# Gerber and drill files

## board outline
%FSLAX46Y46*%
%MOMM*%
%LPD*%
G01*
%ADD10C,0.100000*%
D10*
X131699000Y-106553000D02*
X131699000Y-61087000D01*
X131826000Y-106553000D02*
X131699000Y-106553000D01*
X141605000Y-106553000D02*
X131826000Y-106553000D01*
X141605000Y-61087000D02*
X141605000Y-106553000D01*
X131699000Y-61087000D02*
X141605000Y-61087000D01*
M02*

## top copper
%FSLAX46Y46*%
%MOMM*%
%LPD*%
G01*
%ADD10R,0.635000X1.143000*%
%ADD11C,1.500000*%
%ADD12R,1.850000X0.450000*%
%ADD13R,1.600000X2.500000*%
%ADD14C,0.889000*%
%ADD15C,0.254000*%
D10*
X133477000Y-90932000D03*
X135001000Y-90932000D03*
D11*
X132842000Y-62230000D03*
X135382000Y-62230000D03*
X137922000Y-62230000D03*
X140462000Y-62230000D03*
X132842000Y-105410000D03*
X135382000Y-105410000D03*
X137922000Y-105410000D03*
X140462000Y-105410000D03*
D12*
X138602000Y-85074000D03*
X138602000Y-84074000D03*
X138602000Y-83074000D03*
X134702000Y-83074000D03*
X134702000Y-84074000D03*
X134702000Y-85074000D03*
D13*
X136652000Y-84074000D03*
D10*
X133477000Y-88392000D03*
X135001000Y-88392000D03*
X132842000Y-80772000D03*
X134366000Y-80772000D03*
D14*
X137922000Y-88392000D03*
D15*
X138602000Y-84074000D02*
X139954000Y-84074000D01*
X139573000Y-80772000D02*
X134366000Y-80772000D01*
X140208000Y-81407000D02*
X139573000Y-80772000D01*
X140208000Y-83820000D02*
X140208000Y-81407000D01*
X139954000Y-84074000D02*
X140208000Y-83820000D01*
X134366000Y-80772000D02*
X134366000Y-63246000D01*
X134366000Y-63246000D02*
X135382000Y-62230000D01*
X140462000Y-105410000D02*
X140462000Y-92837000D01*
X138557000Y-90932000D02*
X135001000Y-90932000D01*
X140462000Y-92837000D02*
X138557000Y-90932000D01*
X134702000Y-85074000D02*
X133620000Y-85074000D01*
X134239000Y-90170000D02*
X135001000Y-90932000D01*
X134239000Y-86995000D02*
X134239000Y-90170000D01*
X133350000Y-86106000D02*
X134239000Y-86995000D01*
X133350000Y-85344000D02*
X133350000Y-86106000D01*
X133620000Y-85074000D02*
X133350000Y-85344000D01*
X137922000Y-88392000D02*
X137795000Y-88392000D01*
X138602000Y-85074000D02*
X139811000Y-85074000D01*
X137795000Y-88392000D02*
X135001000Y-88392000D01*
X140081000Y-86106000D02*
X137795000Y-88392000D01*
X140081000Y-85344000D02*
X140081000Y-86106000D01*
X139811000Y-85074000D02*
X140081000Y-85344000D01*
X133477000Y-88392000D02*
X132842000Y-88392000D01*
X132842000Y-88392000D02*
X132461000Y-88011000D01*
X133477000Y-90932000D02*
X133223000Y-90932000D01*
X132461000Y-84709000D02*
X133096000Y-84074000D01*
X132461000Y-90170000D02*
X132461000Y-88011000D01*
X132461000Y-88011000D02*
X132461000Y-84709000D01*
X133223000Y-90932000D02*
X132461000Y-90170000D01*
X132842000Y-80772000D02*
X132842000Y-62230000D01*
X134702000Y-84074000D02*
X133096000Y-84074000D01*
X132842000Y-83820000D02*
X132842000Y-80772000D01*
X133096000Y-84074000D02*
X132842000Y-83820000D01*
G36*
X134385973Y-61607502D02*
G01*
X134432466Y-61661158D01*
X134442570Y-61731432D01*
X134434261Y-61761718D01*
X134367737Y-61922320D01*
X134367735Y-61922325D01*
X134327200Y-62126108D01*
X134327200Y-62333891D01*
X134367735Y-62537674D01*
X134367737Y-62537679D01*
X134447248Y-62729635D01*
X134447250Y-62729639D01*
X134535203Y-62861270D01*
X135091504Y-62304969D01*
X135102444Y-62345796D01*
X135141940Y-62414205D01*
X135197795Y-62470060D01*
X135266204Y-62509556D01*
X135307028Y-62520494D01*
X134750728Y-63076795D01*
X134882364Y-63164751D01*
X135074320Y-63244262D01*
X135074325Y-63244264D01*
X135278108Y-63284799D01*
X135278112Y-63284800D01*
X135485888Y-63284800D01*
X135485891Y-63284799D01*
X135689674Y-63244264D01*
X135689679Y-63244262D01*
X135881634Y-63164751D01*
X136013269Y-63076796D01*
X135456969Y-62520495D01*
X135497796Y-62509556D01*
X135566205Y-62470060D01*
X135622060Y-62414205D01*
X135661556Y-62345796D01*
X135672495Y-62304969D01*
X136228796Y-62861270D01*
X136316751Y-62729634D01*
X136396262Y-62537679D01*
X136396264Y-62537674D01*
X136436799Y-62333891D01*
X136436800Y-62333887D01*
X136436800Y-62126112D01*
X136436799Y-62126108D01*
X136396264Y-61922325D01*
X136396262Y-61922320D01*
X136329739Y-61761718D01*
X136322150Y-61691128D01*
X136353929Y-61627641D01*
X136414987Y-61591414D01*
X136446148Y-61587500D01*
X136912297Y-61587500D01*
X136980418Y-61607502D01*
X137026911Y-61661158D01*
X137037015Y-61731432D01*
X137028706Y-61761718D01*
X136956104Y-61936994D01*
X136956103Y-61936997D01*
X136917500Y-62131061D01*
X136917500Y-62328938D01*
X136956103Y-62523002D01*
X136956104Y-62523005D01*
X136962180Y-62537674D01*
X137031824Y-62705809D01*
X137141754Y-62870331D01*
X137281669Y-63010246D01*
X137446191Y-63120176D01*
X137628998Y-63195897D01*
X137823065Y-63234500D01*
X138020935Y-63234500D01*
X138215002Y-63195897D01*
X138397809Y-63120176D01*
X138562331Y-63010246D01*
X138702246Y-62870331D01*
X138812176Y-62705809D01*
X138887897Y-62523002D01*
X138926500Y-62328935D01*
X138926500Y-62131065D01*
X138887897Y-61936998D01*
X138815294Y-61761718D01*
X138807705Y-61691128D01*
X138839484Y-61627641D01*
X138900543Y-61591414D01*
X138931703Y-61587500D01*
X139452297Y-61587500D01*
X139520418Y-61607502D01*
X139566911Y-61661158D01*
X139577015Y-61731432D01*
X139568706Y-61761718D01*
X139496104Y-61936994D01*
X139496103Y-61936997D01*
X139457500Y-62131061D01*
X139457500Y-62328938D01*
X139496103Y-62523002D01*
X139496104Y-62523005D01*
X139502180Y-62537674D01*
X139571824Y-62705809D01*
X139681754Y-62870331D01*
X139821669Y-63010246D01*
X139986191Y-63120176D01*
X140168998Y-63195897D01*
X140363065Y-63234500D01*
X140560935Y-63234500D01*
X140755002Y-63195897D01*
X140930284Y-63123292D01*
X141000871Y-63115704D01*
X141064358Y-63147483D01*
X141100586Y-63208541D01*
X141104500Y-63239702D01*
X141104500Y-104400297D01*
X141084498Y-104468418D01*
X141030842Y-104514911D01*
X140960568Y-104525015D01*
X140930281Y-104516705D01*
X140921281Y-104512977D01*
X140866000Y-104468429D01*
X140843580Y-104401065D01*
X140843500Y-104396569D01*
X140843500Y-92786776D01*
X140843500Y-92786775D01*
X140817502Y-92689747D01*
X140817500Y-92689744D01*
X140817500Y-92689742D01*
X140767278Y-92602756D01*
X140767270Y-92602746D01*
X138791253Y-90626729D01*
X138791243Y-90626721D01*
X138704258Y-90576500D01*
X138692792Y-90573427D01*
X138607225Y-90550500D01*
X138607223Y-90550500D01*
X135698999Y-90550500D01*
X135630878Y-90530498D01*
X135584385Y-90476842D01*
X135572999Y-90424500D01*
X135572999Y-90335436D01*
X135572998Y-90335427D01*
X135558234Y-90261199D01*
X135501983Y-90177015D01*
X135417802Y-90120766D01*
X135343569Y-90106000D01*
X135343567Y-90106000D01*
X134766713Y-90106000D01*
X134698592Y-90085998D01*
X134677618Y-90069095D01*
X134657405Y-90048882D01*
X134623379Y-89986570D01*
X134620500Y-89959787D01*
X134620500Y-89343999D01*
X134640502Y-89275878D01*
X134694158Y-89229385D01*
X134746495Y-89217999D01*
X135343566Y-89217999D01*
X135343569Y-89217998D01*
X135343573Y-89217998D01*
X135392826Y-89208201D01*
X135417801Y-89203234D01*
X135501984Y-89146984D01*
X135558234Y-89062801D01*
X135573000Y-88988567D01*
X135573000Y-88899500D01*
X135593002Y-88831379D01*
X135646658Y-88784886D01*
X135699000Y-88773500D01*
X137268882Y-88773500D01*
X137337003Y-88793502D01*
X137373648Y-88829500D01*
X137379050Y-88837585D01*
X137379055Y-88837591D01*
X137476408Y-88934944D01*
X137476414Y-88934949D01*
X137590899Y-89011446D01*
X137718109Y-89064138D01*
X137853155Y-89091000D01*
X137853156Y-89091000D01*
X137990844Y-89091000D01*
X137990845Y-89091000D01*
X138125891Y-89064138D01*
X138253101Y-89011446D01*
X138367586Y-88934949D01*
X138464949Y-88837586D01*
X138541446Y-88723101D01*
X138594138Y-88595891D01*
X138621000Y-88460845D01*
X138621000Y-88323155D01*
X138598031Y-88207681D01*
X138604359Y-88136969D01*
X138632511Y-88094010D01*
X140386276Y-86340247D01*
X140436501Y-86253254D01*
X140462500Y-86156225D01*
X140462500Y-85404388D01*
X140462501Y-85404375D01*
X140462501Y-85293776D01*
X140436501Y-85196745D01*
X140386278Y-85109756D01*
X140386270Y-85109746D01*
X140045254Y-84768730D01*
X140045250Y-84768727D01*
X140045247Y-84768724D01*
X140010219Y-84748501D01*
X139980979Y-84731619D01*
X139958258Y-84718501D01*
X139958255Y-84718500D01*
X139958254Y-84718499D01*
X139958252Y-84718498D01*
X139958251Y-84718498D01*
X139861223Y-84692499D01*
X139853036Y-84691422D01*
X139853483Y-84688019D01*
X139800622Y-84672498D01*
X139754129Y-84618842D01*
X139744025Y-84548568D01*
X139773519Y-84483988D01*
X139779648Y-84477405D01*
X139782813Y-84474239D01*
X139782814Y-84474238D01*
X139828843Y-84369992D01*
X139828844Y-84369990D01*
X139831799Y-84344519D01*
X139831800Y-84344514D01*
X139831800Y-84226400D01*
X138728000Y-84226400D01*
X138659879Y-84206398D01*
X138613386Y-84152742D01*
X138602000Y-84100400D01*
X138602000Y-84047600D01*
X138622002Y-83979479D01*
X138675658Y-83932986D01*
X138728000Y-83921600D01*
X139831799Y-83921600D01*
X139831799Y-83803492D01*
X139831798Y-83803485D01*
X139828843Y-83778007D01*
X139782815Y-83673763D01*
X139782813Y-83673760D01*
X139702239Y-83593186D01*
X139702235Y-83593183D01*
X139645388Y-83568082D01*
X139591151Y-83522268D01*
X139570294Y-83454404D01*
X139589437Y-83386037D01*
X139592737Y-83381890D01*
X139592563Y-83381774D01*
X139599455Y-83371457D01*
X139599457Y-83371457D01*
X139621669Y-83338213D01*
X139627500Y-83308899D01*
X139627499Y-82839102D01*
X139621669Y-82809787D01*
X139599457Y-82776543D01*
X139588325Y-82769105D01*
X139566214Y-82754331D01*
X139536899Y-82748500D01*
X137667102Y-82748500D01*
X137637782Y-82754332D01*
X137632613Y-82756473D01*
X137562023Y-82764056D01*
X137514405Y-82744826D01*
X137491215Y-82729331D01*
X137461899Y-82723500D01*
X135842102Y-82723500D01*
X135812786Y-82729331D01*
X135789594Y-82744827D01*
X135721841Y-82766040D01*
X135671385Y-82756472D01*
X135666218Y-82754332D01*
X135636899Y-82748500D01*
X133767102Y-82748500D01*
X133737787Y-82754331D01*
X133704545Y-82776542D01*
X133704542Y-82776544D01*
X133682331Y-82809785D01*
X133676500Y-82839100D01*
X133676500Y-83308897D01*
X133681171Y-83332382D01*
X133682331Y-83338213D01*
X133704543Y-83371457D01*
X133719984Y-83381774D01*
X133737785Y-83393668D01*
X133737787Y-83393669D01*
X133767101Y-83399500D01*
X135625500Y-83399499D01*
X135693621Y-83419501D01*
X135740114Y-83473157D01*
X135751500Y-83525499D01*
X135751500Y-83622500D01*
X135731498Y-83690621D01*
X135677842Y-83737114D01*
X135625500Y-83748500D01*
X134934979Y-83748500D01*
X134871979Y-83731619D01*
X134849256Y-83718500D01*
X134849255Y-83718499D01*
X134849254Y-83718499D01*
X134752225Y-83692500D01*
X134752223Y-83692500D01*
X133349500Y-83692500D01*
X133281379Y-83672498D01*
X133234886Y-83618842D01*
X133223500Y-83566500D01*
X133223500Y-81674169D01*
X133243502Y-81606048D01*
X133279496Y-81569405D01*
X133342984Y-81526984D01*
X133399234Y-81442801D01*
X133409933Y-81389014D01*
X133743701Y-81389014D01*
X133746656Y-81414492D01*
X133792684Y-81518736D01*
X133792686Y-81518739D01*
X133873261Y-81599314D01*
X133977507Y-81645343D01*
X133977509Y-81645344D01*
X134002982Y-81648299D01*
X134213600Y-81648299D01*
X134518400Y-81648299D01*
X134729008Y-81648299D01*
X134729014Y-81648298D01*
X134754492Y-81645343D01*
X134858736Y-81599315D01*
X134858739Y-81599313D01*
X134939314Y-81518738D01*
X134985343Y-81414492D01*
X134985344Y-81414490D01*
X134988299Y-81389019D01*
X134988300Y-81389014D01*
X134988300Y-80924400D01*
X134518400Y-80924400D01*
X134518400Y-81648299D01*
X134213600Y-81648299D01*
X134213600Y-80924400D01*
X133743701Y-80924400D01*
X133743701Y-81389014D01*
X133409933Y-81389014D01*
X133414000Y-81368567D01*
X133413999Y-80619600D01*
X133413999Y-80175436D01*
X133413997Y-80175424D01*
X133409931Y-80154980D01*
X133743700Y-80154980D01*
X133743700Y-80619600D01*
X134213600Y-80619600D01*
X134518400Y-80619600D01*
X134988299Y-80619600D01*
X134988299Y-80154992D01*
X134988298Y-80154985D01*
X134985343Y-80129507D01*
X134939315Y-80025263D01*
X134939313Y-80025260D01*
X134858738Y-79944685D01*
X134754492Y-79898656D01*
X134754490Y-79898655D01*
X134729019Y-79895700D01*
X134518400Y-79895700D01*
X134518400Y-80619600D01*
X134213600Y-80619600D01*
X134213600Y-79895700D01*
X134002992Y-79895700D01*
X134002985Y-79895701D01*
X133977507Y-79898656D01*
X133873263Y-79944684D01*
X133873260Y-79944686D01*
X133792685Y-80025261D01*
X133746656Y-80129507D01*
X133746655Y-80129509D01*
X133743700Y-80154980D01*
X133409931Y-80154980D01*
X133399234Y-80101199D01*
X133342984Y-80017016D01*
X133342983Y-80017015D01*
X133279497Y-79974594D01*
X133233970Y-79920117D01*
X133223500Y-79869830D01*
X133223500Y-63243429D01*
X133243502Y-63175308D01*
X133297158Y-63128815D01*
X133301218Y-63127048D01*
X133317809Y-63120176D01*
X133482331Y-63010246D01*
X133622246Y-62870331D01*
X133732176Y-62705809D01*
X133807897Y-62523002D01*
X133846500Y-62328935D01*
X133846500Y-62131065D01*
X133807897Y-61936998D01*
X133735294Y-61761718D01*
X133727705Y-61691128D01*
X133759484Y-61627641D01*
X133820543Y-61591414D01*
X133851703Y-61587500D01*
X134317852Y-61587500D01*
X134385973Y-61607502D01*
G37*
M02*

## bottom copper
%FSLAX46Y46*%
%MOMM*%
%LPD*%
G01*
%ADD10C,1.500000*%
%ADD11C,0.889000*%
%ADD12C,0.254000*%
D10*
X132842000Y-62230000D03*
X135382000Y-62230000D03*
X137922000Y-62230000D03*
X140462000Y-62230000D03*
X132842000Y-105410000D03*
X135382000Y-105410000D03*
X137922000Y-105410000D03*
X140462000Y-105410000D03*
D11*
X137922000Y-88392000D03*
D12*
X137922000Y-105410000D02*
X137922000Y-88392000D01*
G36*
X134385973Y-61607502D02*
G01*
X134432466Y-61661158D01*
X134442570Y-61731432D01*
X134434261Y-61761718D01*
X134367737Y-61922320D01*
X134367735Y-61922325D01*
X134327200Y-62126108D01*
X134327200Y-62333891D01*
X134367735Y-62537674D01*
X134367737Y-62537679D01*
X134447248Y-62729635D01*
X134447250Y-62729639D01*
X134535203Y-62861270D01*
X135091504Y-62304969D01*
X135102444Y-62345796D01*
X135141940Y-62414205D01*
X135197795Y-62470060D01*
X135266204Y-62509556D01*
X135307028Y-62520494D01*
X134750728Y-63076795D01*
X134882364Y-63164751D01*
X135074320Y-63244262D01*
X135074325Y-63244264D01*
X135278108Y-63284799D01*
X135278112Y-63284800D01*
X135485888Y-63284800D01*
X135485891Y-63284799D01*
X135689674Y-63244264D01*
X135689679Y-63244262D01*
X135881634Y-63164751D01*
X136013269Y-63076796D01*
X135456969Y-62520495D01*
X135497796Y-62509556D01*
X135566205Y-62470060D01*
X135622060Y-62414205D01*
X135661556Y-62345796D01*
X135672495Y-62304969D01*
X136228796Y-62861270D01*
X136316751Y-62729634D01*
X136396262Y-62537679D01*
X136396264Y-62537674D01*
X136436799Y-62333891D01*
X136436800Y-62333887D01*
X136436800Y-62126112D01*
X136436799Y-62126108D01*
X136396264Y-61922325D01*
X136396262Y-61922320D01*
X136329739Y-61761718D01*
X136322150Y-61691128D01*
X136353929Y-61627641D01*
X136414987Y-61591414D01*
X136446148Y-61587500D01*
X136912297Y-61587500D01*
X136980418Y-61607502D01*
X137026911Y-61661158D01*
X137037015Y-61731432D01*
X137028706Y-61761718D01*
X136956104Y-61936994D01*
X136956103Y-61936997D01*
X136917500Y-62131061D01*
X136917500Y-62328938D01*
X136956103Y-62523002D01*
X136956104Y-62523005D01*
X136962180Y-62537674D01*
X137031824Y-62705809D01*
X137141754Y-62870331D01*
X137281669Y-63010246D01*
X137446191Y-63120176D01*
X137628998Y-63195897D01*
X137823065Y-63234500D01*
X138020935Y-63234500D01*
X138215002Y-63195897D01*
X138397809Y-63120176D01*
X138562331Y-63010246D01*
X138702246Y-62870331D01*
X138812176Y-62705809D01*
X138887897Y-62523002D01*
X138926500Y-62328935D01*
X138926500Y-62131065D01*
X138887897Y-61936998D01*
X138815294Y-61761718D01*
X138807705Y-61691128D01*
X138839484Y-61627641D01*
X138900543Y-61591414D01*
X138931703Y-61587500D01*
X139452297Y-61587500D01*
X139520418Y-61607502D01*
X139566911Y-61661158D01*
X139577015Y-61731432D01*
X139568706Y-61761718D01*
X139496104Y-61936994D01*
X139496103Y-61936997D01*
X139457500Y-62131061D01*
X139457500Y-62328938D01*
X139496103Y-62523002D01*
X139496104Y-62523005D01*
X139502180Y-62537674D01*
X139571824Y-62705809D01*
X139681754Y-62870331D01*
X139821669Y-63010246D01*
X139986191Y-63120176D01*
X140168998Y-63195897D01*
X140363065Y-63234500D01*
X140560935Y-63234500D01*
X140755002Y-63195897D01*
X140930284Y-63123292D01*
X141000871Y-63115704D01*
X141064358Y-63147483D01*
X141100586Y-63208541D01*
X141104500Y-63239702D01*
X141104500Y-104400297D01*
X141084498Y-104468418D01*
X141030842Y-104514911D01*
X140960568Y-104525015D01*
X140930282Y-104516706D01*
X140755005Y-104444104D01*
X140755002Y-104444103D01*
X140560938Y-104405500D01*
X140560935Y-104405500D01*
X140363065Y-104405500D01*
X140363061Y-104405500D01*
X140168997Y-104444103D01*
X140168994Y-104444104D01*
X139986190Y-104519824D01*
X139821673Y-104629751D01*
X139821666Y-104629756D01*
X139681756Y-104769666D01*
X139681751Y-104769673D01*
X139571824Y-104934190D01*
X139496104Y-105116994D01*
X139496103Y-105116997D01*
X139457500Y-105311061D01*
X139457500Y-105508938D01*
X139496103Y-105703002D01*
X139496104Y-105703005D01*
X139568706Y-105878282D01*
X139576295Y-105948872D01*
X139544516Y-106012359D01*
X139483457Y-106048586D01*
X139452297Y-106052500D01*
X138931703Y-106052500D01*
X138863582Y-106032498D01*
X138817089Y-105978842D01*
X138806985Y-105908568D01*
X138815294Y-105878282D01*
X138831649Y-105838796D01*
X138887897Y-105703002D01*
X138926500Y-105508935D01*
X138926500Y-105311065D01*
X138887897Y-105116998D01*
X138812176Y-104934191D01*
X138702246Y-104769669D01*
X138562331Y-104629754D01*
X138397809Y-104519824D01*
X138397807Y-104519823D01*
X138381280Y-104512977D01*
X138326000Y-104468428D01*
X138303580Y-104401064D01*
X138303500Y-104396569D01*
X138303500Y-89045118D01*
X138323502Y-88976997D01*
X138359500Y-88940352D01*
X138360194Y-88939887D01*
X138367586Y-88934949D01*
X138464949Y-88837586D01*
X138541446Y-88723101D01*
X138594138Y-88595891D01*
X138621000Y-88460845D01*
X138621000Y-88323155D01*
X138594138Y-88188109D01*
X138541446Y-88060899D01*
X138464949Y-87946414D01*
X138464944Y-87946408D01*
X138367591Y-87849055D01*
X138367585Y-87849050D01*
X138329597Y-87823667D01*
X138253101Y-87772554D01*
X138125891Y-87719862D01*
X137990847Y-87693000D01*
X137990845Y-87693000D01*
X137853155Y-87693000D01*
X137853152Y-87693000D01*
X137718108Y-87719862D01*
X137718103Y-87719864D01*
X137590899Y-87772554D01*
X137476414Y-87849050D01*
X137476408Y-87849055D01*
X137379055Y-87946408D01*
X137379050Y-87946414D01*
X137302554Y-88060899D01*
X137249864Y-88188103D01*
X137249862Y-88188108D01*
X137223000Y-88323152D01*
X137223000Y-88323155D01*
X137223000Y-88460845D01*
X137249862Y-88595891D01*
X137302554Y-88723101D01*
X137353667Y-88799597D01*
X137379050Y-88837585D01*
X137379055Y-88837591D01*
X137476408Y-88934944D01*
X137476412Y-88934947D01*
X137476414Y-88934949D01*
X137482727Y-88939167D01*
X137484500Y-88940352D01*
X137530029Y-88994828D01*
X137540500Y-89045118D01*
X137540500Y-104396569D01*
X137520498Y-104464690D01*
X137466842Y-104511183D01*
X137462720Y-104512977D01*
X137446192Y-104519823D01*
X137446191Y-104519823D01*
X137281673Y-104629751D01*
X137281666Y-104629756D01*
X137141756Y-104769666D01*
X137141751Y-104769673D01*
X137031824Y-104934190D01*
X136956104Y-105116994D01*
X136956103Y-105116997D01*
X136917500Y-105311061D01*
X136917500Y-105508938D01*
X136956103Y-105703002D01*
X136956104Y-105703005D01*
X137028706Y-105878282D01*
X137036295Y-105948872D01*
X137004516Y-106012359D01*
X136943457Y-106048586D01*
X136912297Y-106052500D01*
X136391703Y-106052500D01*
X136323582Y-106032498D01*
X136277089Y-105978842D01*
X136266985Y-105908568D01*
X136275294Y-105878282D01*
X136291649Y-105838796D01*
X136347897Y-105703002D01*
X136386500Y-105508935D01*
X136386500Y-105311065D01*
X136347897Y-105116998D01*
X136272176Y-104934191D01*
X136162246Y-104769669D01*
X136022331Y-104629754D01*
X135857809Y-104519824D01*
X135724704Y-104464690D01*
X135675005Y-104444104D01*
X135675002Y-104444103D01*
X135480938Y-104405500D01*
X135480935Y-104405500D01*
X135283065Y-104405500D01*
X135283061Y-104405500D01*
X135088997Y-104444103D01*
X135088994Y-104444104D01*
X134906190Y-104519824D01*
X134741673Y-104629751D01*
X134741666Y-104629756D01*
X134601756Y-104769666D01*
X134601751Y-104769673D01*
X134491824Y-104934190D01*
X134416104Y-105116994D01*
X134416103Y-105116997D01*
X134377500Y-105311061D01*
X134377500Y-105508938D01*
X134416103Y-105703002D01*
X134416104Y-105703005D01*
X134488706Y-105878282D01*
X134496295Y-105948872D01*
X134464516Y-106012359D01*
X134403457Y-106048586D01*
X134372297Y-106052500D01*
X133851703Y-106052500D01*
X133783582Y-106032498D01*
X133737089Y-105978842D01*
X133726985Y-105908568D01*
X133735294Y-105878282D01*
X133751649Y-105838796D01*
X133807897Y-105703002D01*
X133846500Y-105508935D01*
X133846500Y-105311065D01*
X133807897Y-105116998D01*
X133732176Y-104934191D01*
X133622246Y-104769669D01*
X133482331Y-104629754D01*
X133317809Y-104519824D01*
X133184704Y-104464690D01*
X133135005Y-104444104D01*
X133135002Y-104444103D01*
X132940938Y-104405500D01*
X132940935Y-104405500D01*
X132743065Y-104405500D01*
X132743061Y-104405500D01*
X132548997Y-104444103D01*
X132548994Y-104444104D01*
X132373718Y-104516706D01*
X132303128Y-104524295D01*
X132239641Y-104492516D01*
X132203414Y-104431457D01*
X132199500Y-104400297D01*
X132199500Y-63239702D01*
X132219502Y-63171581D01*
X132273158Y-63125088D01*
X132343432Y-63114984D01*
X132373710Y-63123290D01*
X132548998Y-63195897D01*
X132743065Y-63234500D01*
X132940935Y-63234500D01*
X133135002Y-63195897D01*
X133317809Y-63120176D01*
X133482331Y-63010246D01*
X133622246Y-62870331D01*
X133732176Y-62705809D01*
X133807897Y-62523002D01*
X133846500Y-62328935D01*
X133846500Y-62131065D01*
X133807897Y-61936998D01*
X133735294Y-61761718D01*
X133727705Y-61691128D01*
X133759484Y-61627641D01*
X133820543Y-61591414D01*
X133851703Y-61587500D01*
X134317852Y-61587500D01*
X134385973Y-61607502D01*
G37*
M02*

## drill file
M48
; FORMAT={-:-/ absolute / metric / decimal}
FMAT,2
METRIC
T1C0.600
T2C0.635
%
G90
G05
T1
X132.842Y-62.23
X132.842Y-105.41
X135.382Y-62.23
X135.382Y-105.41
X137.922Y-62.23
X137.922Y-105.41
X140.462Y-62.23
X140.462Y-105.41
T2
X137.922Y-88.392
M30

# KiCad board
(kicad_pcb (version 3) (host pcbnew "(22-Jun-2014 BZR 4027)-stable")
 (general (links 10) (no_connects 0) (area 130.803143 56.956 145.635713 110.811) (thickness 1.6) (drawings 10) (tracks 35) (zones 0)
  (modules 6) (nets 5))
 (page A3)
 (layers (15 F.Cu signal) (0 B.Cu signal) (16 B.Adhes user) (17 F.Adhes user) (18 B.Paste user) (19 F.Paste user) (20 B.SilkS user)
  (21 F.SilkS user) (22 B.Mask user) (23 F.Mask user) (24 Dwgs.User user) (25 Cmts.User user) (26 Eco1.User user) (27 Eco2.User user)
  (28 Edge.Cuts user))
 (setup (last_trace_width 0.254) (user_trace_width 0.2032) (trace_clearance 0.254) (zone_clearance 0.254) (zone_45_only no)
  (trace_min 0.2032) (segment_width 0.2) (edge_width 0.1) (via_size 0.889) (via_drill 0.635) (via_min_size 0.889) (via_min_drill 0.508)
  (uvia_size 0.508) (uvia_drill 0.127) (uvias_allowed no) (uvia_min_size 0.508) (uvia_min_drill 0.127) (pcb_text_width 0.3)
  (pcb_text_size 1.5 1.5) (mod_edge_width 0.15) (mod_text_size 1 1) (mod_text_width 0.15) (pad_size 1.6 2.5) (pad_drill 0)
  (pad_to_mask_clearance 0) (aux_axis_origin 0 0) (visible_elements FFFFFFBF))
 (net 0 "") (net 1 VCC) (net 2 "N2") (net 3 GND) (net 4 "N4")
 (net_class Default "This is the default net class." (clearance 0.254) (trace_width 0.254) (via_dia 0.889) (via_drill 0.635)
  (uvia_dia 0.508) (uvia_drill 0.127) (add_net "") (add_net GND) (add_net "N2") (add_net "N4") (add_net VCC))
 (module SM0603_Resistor (layer F.Cu) (at 134.239 90.932)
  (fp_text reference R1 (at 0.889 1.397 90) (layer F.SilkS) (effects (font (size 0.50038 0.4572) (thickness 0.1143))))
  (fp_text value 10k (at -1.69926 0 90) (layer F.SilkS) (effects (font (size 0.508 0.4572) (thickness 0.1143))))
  (pad 1 smd rect (at -0.762 0) (size 0.635 1.143) (layers F.Cu F.Paste F.Mask) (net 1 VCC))
  (pad 2 smd rect (at 0.762 0) (size 0.635 1.143) (layers F.Cu F.Paste F.Mask) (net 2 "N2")))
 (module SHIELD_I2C (layer F.Cu) (at 136.652 83.82)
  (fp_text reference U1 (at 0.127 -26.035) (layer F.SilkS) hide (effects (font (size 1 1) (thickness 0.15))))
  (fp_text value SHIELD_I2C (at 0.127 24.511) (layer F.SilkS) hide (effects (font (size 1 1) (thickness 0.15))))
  (pad 1 thru_hole circle (at -3.81 -21.59) (size 1.5 1.5) (drill 0.6) (layers *.Cu *.Mask F.SilkS) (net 1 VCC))
  (pad 2 thru_hole circle (at -1.27 -21.59) (size 1.5 1.5) (drill 0.6) (layers *.Cu *.Mask F.SilkS) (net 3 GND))
  (pad 3 thru_hole circle (at 1.27 -21.59) (size 1.5 1.5) (drill 0.6) (layers *.Cu *.Mask F.SilkS))
  (pad 4 thru_hole circle (at 3.81 -21.59) (size 1.5 1.5) (drill 0.6) (layers *.Cu *.Mask F.SilkS))
  (pad 5 thru_hole circle (at -3.81 21.59) (size 1.5 1.5) (drill 0.6) (layers *.Cu *.Mask F.SilkS))
  (pad 6 thru_hole circle (at -1.27 21.59) (size 1.5 1.5) (drill 0.6) (layers *.Cu *.Mask F.SilkS))
  (pad 7 thru_hole circle (at 1.27 21.59) (size 1.5 1.5) (drill 0.6) (layers *.Cu *.Mask F.SilkS) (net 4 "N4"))
  (pad 8 thru_hole circle (at 3.81 21.59) (size 1.5 1.5) (drill 0.6) (layers *.Cu *.Mask F.SilkS) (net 2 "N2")))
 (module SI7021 (layer F.Cu) (at 136.652 84.074 180) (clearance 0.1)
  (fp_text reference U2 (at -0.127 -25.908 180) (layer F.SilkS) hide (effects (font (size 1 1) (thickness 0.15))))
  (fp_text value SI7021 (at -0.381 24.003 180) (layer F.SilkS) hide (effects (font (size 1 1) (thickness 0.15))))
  (pad 1 smd rect (at -1.95 -1 180) (size 1.85 0.45) (layers F.Cu F.Paste F.Mask) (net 4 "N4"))
  (pad 2 smd rect (at -1.95 0 180) (size 1.85 0.45) (layers F.Cu F.Paste F.Mask) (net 3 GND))
  (pad 3 smd rect (at -1.95 1 180) (size 1.85 0.45) (layers F.Cu F.Paste F.Mask))
  (pad 4 smd rect (at 1.95 1 180) (size 1.85 0.45) (layers F.Cu F.Paste F.Mask))
  (pad 5 smd rect (at 1.95 0 180) (size 1.85 0.45) (layers F.Cu F.Paste F.Mask) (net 1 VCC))
  (pad 6 smd rect (at 1.95 -1 180) (size 1.85 0.45) (layers F.Cu F.Paste F.Mask) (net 2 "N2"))
  (pad 7 smd rect (at 0 0 180) (size 1.6 2.5) (layers F.Cu F.Paste F.Mask)))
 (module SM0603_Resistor (layer F.Cu) (at 134.239 88.392)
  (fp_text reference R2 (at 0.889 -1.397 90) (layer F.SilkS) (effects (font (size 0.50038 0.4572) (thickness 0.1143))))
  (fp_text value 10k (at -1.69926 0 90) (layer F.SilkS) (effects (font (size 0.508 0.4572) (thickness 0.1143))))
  (pad 1 smd rect (at -0.762 0) (size 0.635 1.143) (layers F.Cu F.Paste F.Mask) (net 1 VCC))
  (pad 2 smd rect (at 0.762 0) (size 0.635 1.143) (layers F.Cu F.Paste F.Mask) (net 4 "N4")))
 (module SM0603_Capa (layer F.Cu) (at 133.604 80.772)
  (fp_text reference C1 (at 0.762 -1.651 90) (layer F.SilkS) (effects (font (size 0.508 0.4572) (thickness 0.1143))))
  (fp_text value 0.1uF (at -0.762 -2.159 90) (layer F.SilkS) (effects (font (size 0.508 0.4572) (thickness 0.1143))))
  (pad 1 smd rect (at -0.762 0) (size 0.635 1.143) (layers F.Cu F.Paste F.Mask) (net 1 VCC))
  (pad 2 smd rect (at 0.762 0) (size 0.635 1.143) (layers F.Cu F.Paste F.Mask) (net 3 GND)))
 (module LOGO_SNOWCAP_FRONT (layer F.Cu) (at 138.811 71.501 90)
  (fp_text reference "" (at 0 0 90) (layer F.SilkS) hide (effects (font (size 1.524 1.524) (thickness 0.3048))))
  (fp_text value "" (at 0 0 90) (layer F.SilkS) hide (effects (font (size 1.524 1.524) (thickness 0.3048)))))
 (gr_line (start 131.699 106.553) (end 131.699 61.087) (angle 90) (layer Edge.Cuts) (width 0.1))
 (gr_line (start 131.826 106.553) (end 131.699 106.553) (angle 90) (layer Edge.Cuts) (width 0.1))
 (gr_line (start 141.605 106.553) (end 131.826 106.553) (angle 90) (layer Edge.Cuts) (width 0.1))
 (gr_line (start 141.605 61.087) (end 141.605 106.553) (angle 90) (layer Edge.Cuts) (width 0.1))
 (gr_line (start 131.699 61.087) (end 141.605 61.087) (angle 90) (layer Edge.Cuts) (width 0.1))
 (segment (start 138.602 84.074) (end 139.954 84.074) (width 0.254) (layer F.Cu) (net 3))
 (segment (start 139.573 80.772) (end 134.366 80.772) (width 0.254) (layer F.Cu) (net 3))
 (segment (start 140.208 81.407) (end 139.573 80.772) (width 0.254) (layer F.Cu) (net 3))
 (segment (start 140.208 83.82) (end 140.208 81.407) (width 0.254) (layer F.Cu) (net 3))
 (segment (start 139.954 84.074) (end 140.208 83.82) (width 0.254) (layer F.Cu) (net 3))
 (segment (start 134.366 80.772) (end 134.366 63.246) (width 0.254) (layer F.Cu) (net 3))
 (segment (start 134.366 63.246) (end 135.382 62.23) (width 0.254) (layer F.Cu) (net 3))
 (segment (start 140.462 105.41) (end 140.462 92.837) (width 0.254) (layer F.Cu) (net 2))
 (segment (start 138.557 90.932) (end 135.001 90.932) (width 0.254) (layer F.Cu) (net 2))
 (segment (start 140.462 92.837) (end 138.557 90.932) (width 0.254) (layer F.Cu) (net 2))
 (segment (start 134.702 85.074) (end 133.62 85.074) (width 0.254) (layer F.Cu) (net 2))
 (segment (start 134.239 90.17) (end 135.001 90.932) (width 0.254) (layer F.Cu) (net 2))
 (segment (start 134.239 86.995) (end 134.239 90.17) (width 0.254) (layer F.Cu) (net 2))
 (segment (start 133.35 86.106) (end 134.239 86.995) (width 0.254) (layer F.Cu) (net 2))
 (segment (start 133.35 85.344) (end 133.35 86.106) (width 0.254) (layer F.Cu) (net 2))
 (segment (start 133.62 85.074) (end 133.35 85.344) (width 0.254) (layer F.Cu) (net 2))
 (segment (start 137.922 105.41) (end 137.922 88.392) (width 0.254) (layer B.Cu) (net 4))
 (segment (start 137.922 88.392) (end 137.795 88.392) (width 0.254) (layer F.Cu) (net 4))
 (via (at 137.922 88.392) (size 0.889) (layers F.Cu B.Cu) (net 4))
 (segment (start 138.602 85.074) (end 139.811 85.074) (width 0.254) (layer F.Cu) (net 4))
 (segment (start 137.795 88.392) (end 135.001 88.392) (width 0.254) (layer F.Cu) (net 4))
 (segment (start 140.081 86.106) (end 137.795 88.392) (width 0.254) (layer F.Cu) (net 4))
 (segment (start 140.081 85.344) (end 140.081 86.106) (width 0.254) (layer F.Cu) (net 4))
 (segment (start 139.811 85.074) (end 140.081 85.344) (width 0.254) (layer F.Cu) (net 4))
 (segment (start 133.477 88.392) (end 132.842 88.392) (width 0.254) (layer F.Cu) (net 1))
 (segment (start 132.842 88.392) (end 132.461 88.011) (width 0.254) (layer F.Cu) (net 1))
 (segment (start 133.477 90.932) (end 133.223 90.932) (width 0.254) (layer F.Cu) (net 1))
 (segment (start 132.461 84.709) (end 133.096 84.074) (width 0.254) (layer F.Cu) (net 1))
 (segment (start 132.461 90.17) (end 132.461 88.011) (width 0.254) (layer F.Cu) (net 1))
 (segment (start 132.461 88.011) (end 132.461 84.709) (width 0.254) (layer F.Cu) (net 1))
 (segment (start 133.223 90.932) (end 132.461 90.17) (width 0.254) (layer F.Cu) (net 1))
 (segment (start 132.842 80.772) (end 132.842 62.23) (width 0.254) (layer F.Cu) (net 1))
 (segment (start 134.702 84.074) (end 133.096 84.074) (width 0.254) (layer F.Cu) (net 1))
 (segment (start 132.842 83.82) (end 132.842 80.772) (width 0.254) (layer F.Cu) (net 1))
 (segment (start 133.096 84.074) (end 132.842 83.82) (width 0.254) (layer F.Cu) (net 1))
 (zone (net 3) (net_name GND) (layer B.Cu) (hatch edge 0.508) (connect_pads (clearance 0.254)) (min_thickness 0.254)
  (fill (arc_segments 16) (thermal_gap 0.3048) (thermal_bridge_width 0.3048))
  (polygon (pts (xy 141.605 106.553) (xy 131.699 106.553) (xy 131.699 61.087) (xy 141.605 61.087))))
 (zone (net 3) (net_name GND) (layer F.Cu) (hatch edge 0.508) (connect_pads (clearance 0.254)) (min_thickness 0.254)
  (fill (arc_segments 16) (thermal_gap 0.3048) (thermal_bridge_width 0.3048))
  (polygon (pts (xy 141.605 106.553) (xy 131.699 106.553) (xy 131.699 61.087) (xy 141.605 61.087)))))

